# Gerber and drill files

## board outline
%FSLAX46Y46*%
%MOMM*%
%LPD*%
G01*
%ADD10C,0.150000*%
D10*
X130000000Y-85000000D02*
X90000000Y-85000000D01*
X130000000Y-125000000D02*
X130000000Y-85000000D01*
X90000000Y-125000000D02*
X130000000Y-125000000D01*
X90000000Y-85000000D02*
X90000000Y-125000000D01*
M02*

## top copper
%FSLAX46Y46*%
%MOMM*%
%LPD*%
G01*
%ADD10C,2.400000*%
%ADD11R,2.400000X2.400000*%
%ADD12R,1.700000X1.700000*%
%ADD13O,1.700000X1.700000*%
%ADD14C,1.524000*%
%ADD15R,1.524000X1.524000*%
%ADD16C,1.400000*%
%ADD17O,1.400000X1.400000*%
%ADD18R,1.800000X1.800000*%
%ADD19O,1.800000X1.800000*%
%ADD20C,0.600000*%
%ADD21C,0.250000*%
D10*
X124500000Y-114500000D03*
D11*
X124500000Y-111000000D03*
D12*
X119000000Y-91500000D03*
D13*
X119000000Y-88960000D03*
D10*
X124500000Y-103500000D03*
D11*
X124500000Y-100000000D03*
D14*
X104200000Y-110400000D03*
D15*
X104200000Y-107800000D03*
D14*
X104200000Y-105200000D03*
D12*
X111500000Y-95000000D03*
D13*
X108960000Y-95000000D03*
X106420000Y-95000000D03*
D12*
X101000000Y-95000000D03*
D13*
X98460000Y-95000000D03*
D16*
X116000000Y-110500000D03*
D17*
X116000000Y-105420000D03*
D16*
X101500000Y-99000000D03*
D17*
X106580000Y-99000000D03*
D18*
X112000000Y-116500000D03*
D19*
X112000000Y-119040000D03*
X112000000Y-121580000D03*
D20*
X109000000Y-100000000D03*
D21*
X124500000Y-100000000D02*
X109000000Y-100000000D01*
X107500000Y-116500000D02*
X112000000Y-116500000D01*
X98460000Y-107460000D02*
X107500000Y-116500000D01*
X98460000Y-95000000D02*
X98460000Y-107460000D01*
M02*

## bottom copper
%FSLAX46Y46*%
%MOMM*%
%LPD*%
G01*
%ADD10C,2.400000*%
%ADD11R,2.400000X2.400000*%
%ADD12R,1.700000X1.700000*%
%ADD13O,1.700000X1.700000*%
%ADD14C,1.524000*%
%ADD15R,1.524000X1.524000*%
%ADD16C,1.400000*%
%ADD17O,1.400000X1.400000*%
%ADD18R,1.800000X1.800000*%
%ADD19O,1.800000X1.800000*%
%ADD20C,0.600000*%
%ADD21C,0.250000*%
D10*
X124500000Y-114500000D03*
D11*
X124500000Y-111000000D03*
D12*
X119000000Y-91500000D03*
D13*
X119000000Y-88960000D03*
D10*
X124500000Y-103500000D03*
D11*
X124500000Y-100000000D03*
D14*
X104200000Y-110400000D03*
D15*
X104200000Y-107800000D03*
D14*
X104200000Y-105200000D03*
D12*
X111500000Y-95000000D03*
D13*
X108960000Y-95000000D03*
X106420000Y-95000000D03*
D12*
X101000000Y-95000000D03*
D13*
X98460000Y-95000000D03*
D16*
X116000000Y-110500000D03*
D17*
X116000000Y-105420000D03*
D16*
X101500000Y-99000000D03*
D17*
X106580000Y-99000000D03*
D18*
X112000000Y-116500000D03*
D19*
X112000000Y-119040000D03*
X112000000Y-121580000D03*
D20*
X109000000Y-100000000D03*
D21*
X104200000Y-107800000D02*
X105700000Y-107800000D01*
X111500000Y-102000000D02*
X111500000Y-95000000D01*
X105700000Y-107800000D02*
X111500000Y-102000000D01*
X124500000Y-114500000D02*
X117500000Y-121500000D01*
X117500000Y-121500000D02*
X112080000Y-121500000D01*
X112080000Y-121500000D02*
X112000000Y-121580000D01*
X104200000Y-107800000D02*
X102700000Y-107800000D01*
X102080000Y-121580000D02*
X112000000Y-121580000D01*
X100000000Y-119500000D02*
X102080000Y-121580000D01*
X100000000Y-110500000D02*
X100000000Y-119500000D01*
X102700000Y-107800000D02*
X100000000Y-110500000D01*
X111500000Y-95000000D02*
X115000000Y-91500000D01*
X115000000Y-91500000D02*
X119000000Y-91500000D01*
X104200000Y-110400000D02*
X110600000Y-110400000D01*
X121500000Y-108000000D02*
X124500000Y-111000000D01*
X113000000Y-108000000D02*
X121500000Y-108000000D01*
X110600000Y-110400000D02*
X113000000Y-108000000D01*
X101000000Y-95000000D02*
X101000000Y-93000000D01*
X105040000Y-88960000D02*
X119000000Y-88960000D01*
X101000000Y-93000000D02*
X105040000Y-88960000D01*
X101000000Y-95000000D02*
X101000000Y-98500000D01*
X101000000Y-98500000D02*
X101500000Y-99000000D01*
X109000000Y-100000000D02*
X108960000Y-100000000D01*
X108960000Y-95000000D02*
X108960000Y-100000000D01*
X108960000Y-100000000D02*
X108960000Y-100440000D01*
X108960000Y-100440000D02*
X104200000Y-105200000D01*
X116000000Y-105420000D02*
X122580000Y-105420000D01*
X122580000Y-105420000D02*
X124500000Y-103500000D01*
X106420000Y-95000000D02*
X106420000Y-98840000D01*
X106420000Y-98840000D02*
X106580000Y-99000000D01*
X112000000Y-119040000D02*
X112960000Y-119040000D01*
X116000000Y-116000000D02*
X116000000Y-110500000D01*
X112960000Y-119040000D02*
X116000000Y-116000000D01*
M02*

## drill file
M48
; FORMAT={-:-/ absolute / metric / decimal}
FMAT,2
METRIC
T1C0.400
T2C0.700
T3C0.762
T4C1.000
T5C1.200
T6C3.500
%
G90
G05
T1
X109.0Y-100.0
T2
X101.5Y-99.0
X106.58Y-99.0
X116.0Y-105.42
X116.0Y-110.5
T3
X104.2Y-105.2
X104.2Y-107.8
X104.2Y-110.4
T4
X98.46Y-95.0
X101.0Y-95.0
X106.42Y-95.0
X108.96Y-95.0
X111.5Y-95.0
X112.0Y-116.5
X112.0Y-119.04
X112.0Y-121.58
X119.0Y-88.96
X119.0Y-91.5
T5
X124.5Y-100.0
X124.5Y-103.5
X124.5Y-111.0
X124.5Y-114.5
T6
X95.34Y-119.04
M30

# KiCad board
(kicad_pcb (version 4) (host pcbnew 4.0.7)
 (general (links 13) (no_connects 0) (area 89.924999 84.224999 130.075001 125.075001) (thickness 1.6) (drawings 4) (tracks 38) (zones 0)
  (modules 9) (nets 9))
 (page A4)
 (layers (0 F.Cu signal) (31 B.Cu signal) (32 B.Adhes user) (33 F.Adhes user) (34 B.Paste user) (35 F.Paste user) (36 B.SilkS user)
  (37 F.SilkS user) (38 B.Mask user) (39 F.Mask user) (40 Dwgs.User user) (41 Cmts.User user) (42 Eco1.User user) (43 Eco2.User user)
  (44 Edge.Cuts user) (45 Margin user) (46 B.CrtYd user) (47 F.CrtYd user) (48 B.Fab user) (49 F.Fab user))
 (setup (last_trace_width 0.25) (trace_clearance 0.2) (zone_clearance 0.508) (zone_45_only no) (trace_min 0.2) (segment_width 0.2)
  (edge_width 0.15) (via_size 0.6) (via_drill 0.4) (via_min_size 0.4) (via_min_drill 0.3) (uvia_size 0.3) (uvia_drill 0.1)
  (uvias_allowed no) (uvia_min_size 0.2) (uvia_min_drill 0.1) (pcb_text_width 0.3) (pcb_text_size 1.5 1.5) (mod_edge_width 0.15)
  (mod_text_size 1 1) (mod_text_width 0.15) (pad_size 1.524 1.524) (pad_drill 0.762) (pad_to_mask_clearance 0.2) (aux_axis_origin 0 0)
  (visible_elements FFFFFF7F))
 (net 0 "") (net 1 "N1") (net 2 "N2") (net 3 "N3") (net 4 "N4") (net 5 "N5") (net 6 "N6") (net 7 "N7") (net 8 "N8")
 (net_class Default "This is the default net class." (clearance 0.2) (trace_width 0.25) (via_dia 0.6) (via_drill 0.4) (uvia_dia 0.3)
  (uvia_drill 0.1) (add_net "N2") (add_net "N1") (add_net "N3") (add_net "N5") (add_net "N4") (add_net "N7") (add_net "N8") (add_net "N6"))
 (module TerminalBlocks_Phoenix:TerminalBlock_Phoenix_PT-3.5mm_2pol (layer F.Cu) (at 124.5 111 270)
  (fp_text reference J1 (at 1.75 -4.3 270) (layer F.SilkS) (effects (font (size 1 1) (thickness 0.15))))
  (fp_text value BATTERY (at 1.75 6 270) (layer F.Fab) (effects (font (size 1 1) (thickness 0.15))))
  (pad 2 thru_hole circle (at 3.5 0 270) (size 2.4 2.4) (drill 1.2) (layers *.Cu *.Mask) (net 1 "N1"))
  (pad 1 thru_hole rect (at 0 0 270) (size 2.4 2.4) (drill 1.2) (layers *.Cu *.Mask) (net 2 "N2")))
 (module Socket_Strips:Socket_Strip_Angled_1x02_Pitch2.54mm (layer F.Cu) (at 119 91.5 180)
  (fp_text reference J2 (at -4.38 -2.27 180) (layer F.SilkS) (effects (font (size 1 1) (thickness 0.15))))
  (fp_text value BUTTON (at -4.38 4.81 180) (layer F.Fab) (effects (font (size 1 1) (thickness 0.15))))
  (pad 1 thru_hole rect (at 0 0 180) (size 1.7 1.7) (drill 1) (layers *.Cu *.Mask) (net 1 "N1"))
  (pad 2 thru_hole oval (at 0 2.54 180) (size 1.7 1.7) (drill 1) (layers *.Cu *.Mask) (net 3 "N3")))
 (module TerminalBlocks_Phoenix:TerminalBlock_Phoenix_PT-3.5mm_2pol (layer F.Cu) (at 124.5 100 270)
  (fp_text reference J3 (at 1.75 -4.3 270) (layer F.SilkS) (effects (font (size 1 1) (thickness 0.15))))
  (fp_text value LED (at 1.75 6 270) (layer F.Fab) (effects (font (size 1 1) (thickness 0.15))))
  (pad 2 thru_hole circle (at 3.5 0 270) (size 2.4 2.4) (drill 1.2) (layers *.Cu *.Mask) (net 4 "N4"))
  (pad 1 thru_hole rect (at 0 0 270) (size 2.4 2.4) (drill 1.2) (layers *.Cu *.Mask) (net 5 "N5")))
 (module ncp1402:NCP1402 (layer F.Cu) (at 93 112)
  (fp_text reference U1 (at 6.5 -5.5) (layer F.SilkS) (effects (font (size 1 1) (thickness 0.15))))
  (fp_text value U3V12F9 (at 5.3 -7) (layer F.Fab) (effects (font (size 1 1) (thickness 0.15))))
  (pad 1 thru_hole circle (at 11.2 -1.6) (size 1.524 1.524) (drill 0.762) (layers *.Cu *.Mask) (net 2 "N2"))
  (pad 2 thru_hole rect (at 11.2 -4.2) (size 1.524 1.524) (drill 0.762) (layers *.Cu *.Mask) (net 1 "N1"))
  (pad 3 thru_hole circle (at 11.2 -6.8) (size 1.524 1.524) (drill 0.762) (layers *.Cu *.Mask) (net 5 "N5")))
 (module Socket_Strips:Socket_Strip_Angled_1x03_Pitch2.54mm (layer F.Cu) (at 111.5 95 270)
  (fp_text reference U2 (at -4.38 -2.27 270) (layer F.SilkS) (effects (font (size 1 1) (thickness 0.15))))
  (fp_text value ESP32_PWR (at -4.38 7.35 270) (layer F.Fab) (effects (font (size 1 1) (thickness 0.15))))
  (pad 1 thru_hole rect (at 0 0 270) (size 1.7 1.7) (drill 1) (layers *.Cu *.Mask) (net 1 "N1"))
  (pad 2 thru_hole oval (at 0 2.54 270) (size 1.7 1.7) (drill 1) (layers *.Cu *.Mask) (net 5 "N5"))
  (pad 3 thru_hole oval (at 0 5.08 270) (size 1.7 1.7) (drill 1) (layers *.Cu *.Mask) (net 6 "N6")))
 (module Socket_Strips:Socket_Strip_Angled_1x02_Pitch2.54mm (layer F.Cu) (at 101 95 270)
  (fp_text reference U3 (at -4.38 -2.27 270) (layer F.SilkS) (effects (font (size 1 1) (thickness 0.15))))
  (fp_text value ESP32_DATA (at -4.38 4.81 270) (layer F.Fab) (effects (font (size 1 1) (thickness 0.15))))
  (pad 1 thru_hole rect (at 0 0 270) (size 1.7 1.7) (drill 1) (layers *.Cu *.Mask) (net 3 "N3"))
  (pad 2 thru_hole oval (at 0 2.54 270) (size 1.7 1.7) (drill 1) (layers *.Cu *.Mask) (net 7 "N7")))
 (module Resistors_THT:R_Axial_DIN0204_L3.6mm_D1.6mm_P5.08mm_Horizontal (layer F.Cu) (at 116 110.5 90)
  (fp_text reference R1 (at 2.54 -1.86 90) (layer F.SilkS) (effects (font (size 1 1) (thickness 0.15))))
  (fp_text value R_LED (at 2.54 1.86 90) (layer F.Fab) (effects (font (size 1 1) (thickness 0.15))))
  (pad 1 thru_hole circle (at 0 0 90) (size 1.4 1.4) (drill 0.7) (layers *.Cu *.Mask) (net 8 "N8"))
  (pad 2 thru_hole oval (at 5.08 0 90) (size 1.4 1.4) (drill 0.7) (layers *.Cu *.Mask) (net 4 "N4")))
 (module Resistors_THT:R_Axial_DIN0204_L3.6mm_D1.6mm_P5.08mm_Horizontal (layer F.Cu) (at 101.5 99)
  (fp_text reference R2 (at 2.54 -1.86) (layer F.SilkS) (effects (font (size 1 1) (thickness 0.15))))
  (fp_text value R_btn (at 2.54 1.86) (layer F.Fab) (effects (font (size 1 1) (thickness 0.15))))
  (pad 1 thru_hole circle (at 0 0) (size 1.4 1.4) (drill 0.7) (layers *.Cu *.Mask) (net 3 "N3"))
  (pad 2 thru_hole oval (at 5.08 0) (size 1.4 1.4) (drill 0.7) (layers *.Cu *.Mask) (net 6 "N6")))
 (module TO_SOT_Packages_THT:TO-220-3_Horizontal (layer B.Cu) (at 112 116.5 270)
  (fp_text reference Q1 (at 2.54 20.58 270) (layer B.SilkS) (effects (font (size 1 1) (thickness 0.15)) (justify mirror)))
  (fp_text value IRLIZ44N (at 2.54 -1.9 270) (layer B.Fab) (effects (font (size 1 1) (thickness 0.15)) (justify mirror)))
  (pad 0 np_thru_hole oval (at 2.54 16.66 270) (size 3.5 3.5) (drill 3.5) (layers *.Cu *.Mask))
  (pad 1 thru_hole rect (at 0 0 270) (size 1.8 1.8) (drill 1) (layers *.Cu *.Mask) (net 7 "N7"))
  (pad 2 thru_hole oval (at 2.54 0 270) (size 1.8 1.8) (drill 1) (layers *.Cu *.Mask) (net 8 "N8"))
  (pad 3 thru_hole oval (at 5.08 0 270) (size 1.8 1.8) (drill 1) (layers *.Cu *.Mask) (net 1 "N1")))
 (gr_line (start 130 85) (end 90 85) (angle 90) (layer Edge.Cuts) (width 0.15))
 (gr_line (start 130 125) (end 130 85) (angle 90) (layer Edge.Cuts) (width 0.15))
 (gr_line (start 90 125) (end 130 125) (angle 90) (layer Edge.Cuts) (width 0.15))
 (gr_line (start 90 85) (end 90 125) (angle 90) (layer Edge.Cuts) (width 0.15))
 (segment (start 104.2 107.8) (end 105.7 107.8) (width 0.25) (layer B.Cu) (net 1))
 (segment (start 111.5 102) (end 111.5 95) (width 0.25) (layer B.Cu) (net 1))
 (segment (start 105.7 107.8) (end 111.5 102) (width 0.25) (layer B.Cu) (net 1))
 (segment (start 124.5 114.5) (end 117.5 121.5) (width 0.25) (layer B.Cu) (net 1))
 (segment (start 117.5 121.5) (end 112.08 121.5) (width 0.25) (layer B.Cu) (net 1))
 (segment (start 112.08 121.5) (end 112 121.58) (width 0.25) (layer B.Cu) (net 1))
 (segment (start 104.2 107.8) (end 102.7 107.8) (width 0.25) (layer B.Cu) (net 1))
 (segment (start 102.08 121.58) (end 112 121.58) (width 0.25) (layer B.Cu) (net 1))
 (segment (start 100 119.5) (end 102.08 121.58) (width 0.25) (layer B.Cu) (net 1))
 (segment (start 100 110.5) (end 100 119.5) (width 0.25) (layer B.Cu) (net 1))
 (segment (start 102.7 107.8) (end 100 110.5) (width 0.25) (layer B.Cu) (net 1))
 (segment (start 111.5 95) (end 115 91.5) (width 0.25) (layer B.Cu) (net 1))
 (segment (start 115 91.5) (end 119 91.5) (width 0.25) (layer B.Cu) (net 1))
 (segment (start 104.2 110.4) (end 110.6 110.4) (width 0.25) (layer B.Cu) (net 2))
 (segment (start 121.5 108) (end 124.5 111) (width 0.25) (layer B.Cu) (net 2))
 (segment (start 113 108) (end 121.5 108) (width 0.25) (layer B.Cu) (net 2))
 (segment (start 110.6 110.4) (end 113 108) (width 0.25) (layer B.Cu) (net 2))
 (segment (start 101 95) (end 101 93) (width 0.25) (layer B.Cu) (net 3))
 (segment (start 105.04 88.96) (end 119 88.96) (width 0.25) (layer B.Cu) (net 3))
 (segment (start 101 93) (end 105.04 88.96) (width 0.25) (layer B.Cu) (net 3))
 (segment (start 101 95) (end 101 98.5) (width 0.25) (layer B.Cu) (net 3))
 (segment (start 101 98.5) (end 101.5 99) (width 0.25) (layer B.Cu) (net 3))
 (segment (start 124.5 100) (end 109 100) (width 0.25) (layer F.Cu) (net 5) (status 400000))
 (segment (start 109 100) (end 108.96 100) (width 0.25) (layer B.Cu) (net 5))
 (via (at 109 100) (size 0.6) (drill 0.4) (layers F.Cu B.Cu) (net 5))
 (segment (start 108.96 95) (end 108.96 100) (width 0.25) (layer B.Cu) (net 5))
 (segment (start 108.96 100) (end 108.96 100.44) (width 0.25) (layer B.Cu) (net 5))
 (segment (start 108.96 100.44) (end 104.2 105.2) (width 0.25) (layer B.Cu) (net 5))
 (segment (start 116 105.42) (end 122.58 105.42) (width 0.25) (layer B.Cu) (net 4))
 (segment (start 122.58 105.42) (end 124.5 103.5) (width 0.25) (layer B.Cu) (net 4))
 (segment (start 106.42 95) (end 106.42 98.84) (width 0.25) (layer B.Cu) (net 6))
 (segment (start 106.42 98.84) (end 106.58 99) (width 0.25) (layer B.Cu) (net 6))
 (segment (start 107.5 116.5) (end 112 116.5) (width 0.25) (layer F.Cu) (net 7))
 (segment (start 98.46 107.46) (end 107.5 116.5) (width 0.25) (layer F.Cu) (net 7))
 (segment (start 98.46 95) (end 98.46 107.46) (width 0.25) (layer F.Cu) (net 7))
 (segment (start 112 119.04) (end 112.96 119.04) (width 0.25) (layer B.Cu) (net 8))
 (segment (start 116 116) (end 116 110.5) (width 0.25) (layer B.Cu) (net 8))
 (segment (start 112.96 119.04) (end 116 116) (width 0.25) (layer B.Cu) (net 8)))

